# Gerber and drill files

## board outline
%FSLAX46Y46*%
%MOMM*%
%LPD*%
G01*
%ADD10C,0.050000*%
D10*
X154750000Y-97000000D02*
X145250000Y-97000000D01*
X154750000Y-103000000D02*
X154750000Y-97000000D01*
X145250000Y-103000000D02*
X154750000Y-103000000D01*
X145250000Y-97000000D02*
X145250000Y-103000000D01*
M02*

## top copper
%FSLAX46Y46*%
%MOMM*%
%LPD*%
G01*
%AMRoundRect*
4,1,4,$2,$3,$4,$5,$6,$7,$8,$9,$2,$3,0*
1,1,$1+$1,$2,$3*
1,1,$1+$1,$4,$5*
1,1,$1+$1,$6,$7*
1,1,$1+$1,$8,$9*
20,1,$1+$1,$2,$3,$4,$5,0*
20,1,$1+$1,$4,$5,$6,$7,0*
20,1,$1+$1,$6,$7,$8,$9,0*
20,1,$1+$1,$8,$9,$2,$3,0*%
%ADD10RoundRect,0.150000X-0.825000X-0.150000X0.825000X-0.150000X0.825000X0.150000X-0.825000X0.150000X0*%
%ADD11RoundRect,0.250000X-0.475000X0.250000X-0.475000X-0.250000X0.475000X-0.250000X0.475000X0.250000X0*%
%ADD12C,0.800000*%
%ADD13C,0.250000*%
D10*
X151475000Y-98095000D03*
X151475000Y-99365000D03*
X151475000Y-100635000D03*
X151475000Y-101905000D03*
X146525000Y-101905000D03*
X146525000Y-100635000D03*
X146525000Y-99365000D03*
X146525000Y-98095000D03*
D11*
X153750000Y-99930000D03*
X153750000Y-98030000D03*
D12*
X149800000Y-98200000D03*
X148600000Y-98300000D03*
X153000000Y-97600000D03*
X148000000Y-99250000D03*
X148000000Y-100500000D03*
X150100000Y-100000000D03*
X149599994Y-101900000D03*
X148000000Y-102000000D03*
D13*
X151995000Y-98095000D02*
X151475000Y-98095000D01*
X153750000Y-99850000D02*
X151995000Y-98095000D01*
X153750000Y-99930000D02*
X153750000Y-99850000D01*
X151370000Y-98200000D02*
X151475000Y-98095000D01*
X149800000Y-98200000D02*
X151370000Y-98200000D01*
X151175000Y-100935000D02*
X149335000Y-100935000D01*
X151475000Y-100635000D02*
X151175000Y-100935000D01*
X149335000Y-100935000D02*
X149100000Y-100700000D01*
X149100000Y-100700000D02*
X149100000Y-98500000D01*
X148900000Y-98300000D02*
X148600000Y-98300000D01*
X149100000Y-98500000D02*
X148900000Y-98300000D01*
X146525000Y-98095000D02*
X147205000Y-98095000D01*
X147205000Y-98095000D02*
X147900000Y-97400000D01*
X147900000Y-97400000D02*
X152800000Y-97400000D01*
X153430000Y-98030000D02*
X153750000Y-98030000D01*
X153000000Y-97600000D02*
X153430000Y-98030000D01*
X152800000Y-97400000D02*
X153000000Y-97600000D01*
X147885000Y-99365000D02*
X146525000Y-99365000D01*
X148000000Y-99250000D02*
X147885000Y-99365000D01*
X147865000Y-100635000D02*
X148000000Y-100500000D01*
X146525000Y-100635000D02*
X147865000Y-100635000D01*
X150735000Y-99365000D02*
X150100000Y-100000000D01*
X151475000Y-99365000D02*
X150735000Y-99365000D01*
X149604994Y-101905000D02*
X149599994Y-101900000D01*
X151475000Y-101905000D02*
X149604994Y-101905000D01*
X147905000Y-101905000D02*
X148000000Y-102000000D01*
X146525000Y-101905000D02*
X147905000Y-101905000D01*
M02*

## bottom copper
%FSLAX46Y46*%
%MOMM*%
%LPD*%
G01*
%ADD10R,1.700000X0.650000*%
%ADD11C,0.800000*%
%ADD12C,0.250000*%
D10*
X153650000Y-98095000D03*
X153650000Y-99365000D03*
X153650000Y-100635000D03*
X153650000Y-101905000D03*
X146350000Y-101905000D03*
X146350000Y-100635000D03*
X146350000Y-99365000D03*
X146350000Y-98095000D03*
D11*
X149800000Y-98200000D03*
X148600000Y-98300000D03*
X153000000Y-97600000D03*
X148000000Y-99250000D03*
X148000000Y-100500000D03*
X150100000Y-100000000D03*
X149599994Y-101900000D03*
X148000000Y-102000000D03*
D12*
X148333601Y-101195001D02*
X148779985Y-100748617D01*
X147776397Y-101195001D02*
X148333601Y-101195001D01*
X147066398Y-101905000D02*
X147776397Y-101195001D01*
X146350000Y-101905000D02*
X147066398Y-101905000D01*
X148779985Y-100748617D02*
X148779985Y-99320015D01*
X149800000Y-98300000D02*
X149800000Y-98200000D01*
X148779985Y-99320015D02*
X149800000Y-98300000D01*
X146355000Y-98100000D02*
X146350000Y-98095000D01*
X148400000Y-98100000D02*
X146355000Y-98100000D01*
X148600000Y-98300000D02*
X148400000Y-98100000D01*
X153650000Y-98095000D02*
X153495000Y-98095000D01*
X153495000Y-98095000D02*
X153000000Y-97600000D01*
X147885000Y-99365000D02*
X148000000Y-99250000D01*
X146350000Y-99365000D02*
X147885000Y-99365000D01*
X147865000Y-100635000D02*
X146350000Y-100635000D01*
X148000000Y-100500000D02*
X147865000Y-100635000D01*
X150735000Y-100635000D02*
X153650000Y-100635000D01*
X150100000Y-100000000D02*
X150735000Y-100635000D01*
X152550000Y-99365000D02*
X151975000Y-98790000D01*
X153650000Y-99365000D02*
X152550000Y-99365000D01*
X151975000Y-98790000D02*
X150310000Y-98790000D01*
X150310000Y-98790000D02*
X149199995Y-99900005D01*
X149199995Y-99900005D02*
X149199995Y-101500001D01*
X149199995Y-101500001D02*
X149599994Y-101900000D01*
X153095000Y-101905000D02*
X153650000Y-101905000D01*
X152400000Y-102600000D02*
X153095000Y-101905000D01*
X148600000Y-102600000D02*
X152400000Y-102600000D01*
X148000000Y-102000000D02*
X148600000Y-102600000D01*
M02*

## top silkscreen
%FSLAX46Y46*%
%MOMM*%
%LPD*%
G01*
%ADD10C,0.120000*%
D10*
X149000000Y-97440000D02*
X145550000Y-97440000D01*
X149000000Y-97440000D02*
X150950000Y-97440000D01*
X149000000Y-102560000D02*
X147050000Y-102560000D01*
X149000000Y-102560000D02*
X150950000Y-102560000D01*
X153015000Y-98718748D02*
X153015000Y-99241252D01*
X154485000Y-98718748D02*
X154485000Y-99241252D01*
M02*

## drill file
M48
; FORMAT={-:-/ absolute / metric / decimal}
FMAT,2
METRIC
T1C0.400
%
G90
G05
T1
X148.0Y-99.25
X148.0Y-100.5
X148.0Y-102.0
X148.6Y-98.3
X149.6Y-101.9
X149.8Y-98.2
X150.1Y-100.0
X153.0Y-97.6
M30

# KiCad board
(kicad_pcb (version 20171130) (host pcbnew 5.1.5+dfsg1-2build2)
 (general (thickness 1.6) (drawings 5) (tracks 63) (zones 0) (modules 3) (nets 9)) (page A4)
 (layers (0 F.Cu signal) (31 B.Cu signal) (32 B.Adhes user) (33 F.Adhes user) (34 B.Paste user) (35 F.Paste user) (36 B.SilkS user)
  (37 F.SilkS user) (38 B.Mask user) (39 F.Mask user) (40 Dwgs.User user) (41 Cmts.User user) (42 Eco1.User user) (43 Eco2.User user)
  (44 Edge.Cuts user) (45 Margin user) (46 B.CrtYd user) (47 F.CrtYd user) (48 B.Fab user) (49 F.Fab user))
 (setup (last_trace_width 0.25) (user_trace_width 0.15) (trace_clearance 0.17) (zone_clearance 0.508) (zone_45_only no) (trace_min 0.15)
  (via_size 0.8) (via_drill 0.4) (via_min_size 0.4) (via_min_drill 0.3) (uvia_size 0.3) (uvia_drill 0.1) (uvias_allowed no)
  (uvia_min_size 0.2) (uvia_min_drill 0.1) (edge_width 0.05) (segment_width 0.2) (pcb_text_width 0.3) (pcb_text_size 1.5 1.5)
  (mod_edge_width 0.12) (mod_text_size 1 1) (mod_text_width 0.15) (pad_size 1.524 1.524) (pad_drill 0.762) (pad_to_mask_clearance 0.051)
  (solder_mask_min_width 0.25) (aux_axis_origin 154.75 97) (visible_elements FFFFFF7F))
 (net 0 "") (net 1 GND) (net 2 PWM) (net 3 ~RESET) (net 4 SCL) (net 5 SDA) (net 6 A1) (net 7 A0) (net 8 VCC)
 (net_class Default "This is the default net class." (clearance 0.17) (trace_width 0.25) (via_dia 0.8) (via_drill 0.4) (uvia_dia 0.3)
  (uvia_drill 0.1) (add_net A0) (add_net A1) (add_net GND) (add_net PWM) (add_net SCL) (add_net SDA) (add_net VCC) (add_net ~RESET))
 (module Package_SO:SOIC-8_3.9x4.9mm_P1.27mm (layer F.Cu) (at 149 100)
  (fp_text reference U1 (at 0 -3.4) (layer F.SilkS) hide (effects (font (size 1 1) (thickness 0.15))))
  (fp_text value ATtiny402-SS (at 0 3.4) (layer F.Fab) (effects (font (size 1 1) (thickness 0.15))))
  (fp_line (start 0 -2.56) (end -3.45 -2.56) (layer F.SilkS) (width 0.12))
  (fp_line (start 0 -2.56) (end 1.95 -2.56) (layer F.SilkS) (width 0.12))
  (fp_line (start 0 2.56) (end -1.95 2.56) (layer F.SilkS) (width 0.12))
  (fp_line (start 0 2.56) (end 1.95 2.56) (layer F.SilkS) (width 0.12))
  (pad 8 smd roundrect (at 2.475 -1.905) (size 1.95 0.6) (layers F.Cu F.Paste F.Mask) (roundrect_rratio 0.25) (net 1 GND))
  (pad 7 smd roundrect (at 2.475 -0.635) (size 1.95 0.6) (layers F.Cu F.Paste F.Mask) (roundrect_rratio 0.25) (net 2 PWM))
  (pad 6 smd roundrect (at 2.475 0.635) (size 1.95 0.6) (layers F.Cu F.Paste F.Mask) (roundrect_rratio 0.25) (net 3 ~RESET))
  (pad 5 smd roundrect (at 2.475 1.905) (size 1.95 0.6) (layers F.Cu F.Paste F.Mask) (roundrect_rratio 0.25) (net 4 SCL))
  (pad 4 smd roundrect (at -2.475 1.905) (size 1.95 0.6) (layers F.Cu F.Paste F.Mask) (roundrect_rratio 0.25) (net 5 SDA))
  (pad 3 smd roundrect (at -2.475 0.635) (size 1.95 0.6) (layers F.Cu F.Paste F.Mask) (roundrect_rratio 0.25) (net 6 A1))
  (pad 2 smd roundrect (at -2.475 -0.635) (size 1.95 0.6) (layers F.Cu F.Paste F.Mask) (roundrect_rratio 0.25) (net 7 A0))
  (pad 1 smd roundrect (at -2.475 -1.905) (size 1.95 0.6) (layers F.Cu F.Paste F.Mask) (roundrect_rratio 0.25) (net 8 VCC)))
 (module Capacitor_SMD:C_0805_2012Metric (layer F.Cu) (at 153.75 98.98 270)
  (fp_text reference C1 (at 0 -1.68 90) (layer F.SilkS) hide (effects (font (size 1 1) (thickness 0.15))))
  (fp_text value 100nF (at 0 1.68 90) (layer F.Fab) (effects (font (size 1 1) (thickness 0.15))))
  (fp_line (start -0.261252 0.735) (end 0.261252 0.735) (layer F.SilkS) (width 0.12))
  (fp_line (start -0.261252 -0.735) (end 0.261252 -0.735) (layer F.SilkS) (width 0.12))
  (pad 2 smd roundrect (at 0.95 0 270) (size 1 1.45) (layers F.Cu F.Paste F.Mask) (roundrect_rratio 0.25) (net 1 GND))
  (pad 1 smd roundrect (at -0.95 0 270) (size 1 1.45) (layers F.Cu F.Paste F.Mask) (roundrect_rratio 0.25) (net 8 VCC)))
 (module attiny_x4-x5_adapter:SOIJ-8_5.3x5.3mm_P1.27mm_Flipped (layer F.Cu) (at 150 100)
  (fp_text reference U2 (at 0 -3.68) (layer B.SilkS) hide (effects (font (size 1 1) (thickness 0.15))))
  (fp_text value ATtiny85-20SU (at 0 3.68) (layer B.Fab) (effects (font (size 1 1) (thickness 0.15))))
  (pad 8 smd rect (at 3.65 -1.905) (size 1.7 0.65) (layers B.Cu B.Paste B.Mask) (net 8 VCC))
  (pad 7 smd rect (at 3.65 -0.635) (size 1.7 0.65) (layers B.Cu B.Paste B.Mask) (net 4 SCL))
  (pad 6 smd rect (at 3.65 0.635) (size 1.7 0.65) (layers B.Cu B.Paste B.Mask) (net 2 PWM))
  (pad 5 smd rect (at 3.65 1.905) (size 1.7 0.65) (layers B.Cu B.Paste B.Mask) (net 5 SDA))
  (pad 4 smd rect (at -3.65 1.905) (size 1.7 0.65) (layers B.Cu B.Paste B.Mask) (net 1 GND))
  (pad 3 smd rect (at -3.65 0.635) (size 1.7 0.65) (layers B.Cu B.Paste B.Mask) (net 6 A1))
  (pad 2 smd rect (at -3.65 -0.635) (size 1.7 0.65) (layers B.Cu B.Paste B.Mask) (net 7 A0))
  (pad 1 smd rect (at -3.65 -1.905) (size 1.7 0.65) (layers B.Cu B.Paste B.Mask) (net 3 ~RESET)))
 (gr_line (start 154.75 97) (end 145.25 97) (layer Edge.Cuts) (width 0.05))
 (gr_line (start 154.75 103) (end 154.75 97) (layer Edge.Cuts) (width 0.05))
 (gr_line (start 145.25 103) (end 154.75 103) (layer Edge.Cuts) (width 0.05))
 (gr_line (start 145.25 97) (end 145.25 103) (layer Edge.Cuts) (width 0.05))
 (segment (start 151.995 98.095) (end 151.475 98.095) (width 0.25) (layer F.Cu) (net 1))
 (segment (start 153.75 99.85) (end 151.995 98.095) (width 0.25) (layer F.Cu) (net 1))
 (segment (start 153.75 99.93) (end 153.75 99.85) (width 0.25) (layer F.Cu) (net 1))
 (segment (start 148.333601 101.195001) (end 148.779985 100.748617) (width 0.25) (layer B.Cu) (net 1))
 (segment (start 147.776397 101.195001) (end 148.333601 101.195001) (width 0.25) (layer B.Cu) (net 1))
 (segment (start 147.066398 101.905) (end 147.776397 101.195001) (width 0.25) (layer B.Cu) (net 1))
 (segment (start 146.35 101.905) (end 147.066398 101.905) (width 0.25) (layer B.Cu) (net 1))
 (segment (start 148.779985 100.748617) (end 148.779985 99.320015) (width 0.25) (layer B.Cu) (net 1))
 (via (at 149.8 98.2) (size 0.8) (drill 0.4) (layers F.Cu B.Cu) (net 1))
 (segment (start 149.8 98.3) (end 149.8 98.2) (width 0.25) (layer B.Cu) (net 1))
 (segment (start 148.779985 99.320015) (end 149.8 98.3) (width 0.25) (layer B.Cu) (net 1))
 (segment (start 151.37 98.2) (end 151.475 98.095) (width 0.25) (layer F.Cu) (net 1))
 (segment (start 149.8 98.2) (end 151.37 98.2) (width 0.25) (layer F.Cu) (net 1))
 (segment (start 151.175 100.935) (end 149.335 100.935) (width 0.25) (layer F.Cu) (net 3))
 (segment (start 151.475 100.635) (end 151.175 100.935) (width 0.25) (layer F.Cu) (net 3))
 (segment (start 149.335 100.935) (end 149.1 100.7) (width 0.25) (layer F.Cu) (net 3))
 (segment (start 149.1 100.7) (end 149.1 98.5) (width 0.25) (layer F.Cu) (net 3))
 (via (at 148.6 98.3) (size 0.8) (drill 0.4) (layers F.Cu B.Cu) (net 3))
 (segment (start 148.9 98.3) (end 148.6 98.3) (width 0.25) (layer F.Cu) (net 3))
 (segment (start 149.1 98.5) (end 148.9 98.3) (width 0.25) (layer F.Cu) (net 3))
 (segment (start 146.355 98.1) (end 146.35 98.095) (width 0.25) (layer B.Cu) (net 3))
 (segment (start 148.4 98.1) (end 146.355 98.1) (width 0.25) (layer B.Cu) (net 3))
 (segment (start 148.6 98.3) (end 148.4 98.1) (width 0.25) (layer B.Cu) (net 3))
 (segment (start 146.525 98.095) (end 147.205 98.095) (width 0.25) (layer F.Cu) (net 8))
 (segment (start 147.205 98.095) (end 147.9 97.4) (width 0.25) (layer F.Cu) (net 8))
 (segment (start 147.9 97.4) (end 152.8 97.4) (width 0.25) (layer F.Cu) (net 8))
 (segment (start 153.43 98.03) (end 153.75 98.03) (width 0.25) (layer F.Cu) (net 8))
 (segment (start 153.65 98.095) (end 153.495 98.095) (width 0.25) (layer B.Cu) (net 8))
 (segment (start 153.495 98.095) (end 153 97.6) (width 0.25) (layer B.Cu) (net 8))
 (segment (start 153 97.6) (end 153.43 98.03) (width 0.25) (layer F.Cu) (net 8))
 (via (at 153 97.6) (size 0.8) (drill 0.4) (layers F.Cu B.Cu) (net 8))
 (segment (start 152.8 97.4) (end 153 97.6) (width 0.25) (layer F.Cu) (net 8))
 (via (at 148 99.25) (size 0.8) (drill 0.4) (layers F.Cu B.Cu) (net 7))
 (segment (start 147.885 99.365) (end 148 99.25) (width 0.25) (layer B.Cu) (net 7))
 (segment (start 146.35 99.365) (end 147.885 99.365) (width 0.25) (layer B.Cu) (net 7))
 (segment (start 147.885 99.365) (end 146.525 99.365) (width 0.25) (layer F.Cu) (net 7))
 (segment (start 148 99.25) (end 147.885 99.365) (width 0.25) (layer F.Cu) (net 7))
 (segment (start 147.865 100.635) (end 148 100.5) (width 0.25) (layer F.Cu) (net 6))
 (via (at 148 100.5) (size 0.8) (drill 0.4) (layers F.Cu B.Cu) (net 6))
 (segment (start 146.525 100.635) (end 147.865 100.635) (width 0.25) (layer F.Cu) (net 6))
 (segment (start 147.865 100.635) (end 146.35 100.635) (width 0.25) (layer B.Cu) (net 6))
 (segment (start 148 100.5) (end 147.865 100.635) (width 0.25) (layer B.Cu) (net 6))
 (segment (start 150.735 99.365) (end 150.1 100) (width 0.25) (layer F.Cu) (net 2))
 (via (at 150.1 100) (size 0.8) (drill 0.4) (layers F.Cu B.Cu) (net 2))
 (segment (start 151.475 99.365) (end 150.735 99.365) (width 0.25) (layer F.Cu) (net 2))
 (segment (start 150.735 100.635) (end 153.65 100.635) (width 0.25) (layer B.Cu) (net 2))
 (segment (start 150.1 100) (end 150.735 100.635) (width 0.25) (layer B.Cu) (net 2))
 (via (at 149.599994 101.9) (size 0.8) (drill 0.4) (layers F.Cu B.Cu) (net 4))
 (segment (start 152.55 99.365) (end 151.975 98.79) (width 0.25) (layer B.Cu) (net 4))
 (segment (start 149.604994 101.905) (end 149.599994 101.9) (width 0.25) (layer F.Cu) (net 4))
 (segment (start 151.475 101.905) (end 149.604994 101.905) (width 0.25) (layer F.Cu) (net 4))
 (segment (start 153.65 99.365) (end 152.55 99.365) (width 0.25) (layer B.Cu) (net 4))
 (segment (start 151.975 98.79) (end 150.31 98.79) (width 0.25) (layer B.Cu) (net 4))
 (segment (start 150.31 98.79) (end 149.199995 99.900005) (width 0.25) (layer B.Cu) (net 4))
 (segment (start 149.199995 99.900005) (end 149.199995 101.500001) (width 0.25) (layer B.Cu) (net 4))
 (segment (start 149.199995 101.500001) (end 149.599994 101.9) (width 0.25) (layer B.Cu) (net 4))
 (via (at 148 102) (size 0.8) (drill 0.4) (layers F.Cu B.Cu) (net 5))
 (segment (start 147.905 101.905) (end 148 102) (width 0.25) (layer F.Cu) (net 5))
 (segment (start 146.525 101.905) (end 147.905 101.905) (width 0.25) (layer F.Cu) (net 5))
 (segment (start 153.095 101.905) (end 153.65 101.905) (width 0.25) (layer B.Cu) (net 5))
 (segment (start 152.4 102.6) (end 153.095 101.905) (width 0.25) (layer B.Cu) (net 5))
 (segment (start 148.6 102.6) (end 152.4 102.6) (width 0.25) (layer B.Cu) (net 5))
 (segment (start 148 102) (end 148.6 102.6) (width 0.25) (layer B.Cu) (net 5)))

